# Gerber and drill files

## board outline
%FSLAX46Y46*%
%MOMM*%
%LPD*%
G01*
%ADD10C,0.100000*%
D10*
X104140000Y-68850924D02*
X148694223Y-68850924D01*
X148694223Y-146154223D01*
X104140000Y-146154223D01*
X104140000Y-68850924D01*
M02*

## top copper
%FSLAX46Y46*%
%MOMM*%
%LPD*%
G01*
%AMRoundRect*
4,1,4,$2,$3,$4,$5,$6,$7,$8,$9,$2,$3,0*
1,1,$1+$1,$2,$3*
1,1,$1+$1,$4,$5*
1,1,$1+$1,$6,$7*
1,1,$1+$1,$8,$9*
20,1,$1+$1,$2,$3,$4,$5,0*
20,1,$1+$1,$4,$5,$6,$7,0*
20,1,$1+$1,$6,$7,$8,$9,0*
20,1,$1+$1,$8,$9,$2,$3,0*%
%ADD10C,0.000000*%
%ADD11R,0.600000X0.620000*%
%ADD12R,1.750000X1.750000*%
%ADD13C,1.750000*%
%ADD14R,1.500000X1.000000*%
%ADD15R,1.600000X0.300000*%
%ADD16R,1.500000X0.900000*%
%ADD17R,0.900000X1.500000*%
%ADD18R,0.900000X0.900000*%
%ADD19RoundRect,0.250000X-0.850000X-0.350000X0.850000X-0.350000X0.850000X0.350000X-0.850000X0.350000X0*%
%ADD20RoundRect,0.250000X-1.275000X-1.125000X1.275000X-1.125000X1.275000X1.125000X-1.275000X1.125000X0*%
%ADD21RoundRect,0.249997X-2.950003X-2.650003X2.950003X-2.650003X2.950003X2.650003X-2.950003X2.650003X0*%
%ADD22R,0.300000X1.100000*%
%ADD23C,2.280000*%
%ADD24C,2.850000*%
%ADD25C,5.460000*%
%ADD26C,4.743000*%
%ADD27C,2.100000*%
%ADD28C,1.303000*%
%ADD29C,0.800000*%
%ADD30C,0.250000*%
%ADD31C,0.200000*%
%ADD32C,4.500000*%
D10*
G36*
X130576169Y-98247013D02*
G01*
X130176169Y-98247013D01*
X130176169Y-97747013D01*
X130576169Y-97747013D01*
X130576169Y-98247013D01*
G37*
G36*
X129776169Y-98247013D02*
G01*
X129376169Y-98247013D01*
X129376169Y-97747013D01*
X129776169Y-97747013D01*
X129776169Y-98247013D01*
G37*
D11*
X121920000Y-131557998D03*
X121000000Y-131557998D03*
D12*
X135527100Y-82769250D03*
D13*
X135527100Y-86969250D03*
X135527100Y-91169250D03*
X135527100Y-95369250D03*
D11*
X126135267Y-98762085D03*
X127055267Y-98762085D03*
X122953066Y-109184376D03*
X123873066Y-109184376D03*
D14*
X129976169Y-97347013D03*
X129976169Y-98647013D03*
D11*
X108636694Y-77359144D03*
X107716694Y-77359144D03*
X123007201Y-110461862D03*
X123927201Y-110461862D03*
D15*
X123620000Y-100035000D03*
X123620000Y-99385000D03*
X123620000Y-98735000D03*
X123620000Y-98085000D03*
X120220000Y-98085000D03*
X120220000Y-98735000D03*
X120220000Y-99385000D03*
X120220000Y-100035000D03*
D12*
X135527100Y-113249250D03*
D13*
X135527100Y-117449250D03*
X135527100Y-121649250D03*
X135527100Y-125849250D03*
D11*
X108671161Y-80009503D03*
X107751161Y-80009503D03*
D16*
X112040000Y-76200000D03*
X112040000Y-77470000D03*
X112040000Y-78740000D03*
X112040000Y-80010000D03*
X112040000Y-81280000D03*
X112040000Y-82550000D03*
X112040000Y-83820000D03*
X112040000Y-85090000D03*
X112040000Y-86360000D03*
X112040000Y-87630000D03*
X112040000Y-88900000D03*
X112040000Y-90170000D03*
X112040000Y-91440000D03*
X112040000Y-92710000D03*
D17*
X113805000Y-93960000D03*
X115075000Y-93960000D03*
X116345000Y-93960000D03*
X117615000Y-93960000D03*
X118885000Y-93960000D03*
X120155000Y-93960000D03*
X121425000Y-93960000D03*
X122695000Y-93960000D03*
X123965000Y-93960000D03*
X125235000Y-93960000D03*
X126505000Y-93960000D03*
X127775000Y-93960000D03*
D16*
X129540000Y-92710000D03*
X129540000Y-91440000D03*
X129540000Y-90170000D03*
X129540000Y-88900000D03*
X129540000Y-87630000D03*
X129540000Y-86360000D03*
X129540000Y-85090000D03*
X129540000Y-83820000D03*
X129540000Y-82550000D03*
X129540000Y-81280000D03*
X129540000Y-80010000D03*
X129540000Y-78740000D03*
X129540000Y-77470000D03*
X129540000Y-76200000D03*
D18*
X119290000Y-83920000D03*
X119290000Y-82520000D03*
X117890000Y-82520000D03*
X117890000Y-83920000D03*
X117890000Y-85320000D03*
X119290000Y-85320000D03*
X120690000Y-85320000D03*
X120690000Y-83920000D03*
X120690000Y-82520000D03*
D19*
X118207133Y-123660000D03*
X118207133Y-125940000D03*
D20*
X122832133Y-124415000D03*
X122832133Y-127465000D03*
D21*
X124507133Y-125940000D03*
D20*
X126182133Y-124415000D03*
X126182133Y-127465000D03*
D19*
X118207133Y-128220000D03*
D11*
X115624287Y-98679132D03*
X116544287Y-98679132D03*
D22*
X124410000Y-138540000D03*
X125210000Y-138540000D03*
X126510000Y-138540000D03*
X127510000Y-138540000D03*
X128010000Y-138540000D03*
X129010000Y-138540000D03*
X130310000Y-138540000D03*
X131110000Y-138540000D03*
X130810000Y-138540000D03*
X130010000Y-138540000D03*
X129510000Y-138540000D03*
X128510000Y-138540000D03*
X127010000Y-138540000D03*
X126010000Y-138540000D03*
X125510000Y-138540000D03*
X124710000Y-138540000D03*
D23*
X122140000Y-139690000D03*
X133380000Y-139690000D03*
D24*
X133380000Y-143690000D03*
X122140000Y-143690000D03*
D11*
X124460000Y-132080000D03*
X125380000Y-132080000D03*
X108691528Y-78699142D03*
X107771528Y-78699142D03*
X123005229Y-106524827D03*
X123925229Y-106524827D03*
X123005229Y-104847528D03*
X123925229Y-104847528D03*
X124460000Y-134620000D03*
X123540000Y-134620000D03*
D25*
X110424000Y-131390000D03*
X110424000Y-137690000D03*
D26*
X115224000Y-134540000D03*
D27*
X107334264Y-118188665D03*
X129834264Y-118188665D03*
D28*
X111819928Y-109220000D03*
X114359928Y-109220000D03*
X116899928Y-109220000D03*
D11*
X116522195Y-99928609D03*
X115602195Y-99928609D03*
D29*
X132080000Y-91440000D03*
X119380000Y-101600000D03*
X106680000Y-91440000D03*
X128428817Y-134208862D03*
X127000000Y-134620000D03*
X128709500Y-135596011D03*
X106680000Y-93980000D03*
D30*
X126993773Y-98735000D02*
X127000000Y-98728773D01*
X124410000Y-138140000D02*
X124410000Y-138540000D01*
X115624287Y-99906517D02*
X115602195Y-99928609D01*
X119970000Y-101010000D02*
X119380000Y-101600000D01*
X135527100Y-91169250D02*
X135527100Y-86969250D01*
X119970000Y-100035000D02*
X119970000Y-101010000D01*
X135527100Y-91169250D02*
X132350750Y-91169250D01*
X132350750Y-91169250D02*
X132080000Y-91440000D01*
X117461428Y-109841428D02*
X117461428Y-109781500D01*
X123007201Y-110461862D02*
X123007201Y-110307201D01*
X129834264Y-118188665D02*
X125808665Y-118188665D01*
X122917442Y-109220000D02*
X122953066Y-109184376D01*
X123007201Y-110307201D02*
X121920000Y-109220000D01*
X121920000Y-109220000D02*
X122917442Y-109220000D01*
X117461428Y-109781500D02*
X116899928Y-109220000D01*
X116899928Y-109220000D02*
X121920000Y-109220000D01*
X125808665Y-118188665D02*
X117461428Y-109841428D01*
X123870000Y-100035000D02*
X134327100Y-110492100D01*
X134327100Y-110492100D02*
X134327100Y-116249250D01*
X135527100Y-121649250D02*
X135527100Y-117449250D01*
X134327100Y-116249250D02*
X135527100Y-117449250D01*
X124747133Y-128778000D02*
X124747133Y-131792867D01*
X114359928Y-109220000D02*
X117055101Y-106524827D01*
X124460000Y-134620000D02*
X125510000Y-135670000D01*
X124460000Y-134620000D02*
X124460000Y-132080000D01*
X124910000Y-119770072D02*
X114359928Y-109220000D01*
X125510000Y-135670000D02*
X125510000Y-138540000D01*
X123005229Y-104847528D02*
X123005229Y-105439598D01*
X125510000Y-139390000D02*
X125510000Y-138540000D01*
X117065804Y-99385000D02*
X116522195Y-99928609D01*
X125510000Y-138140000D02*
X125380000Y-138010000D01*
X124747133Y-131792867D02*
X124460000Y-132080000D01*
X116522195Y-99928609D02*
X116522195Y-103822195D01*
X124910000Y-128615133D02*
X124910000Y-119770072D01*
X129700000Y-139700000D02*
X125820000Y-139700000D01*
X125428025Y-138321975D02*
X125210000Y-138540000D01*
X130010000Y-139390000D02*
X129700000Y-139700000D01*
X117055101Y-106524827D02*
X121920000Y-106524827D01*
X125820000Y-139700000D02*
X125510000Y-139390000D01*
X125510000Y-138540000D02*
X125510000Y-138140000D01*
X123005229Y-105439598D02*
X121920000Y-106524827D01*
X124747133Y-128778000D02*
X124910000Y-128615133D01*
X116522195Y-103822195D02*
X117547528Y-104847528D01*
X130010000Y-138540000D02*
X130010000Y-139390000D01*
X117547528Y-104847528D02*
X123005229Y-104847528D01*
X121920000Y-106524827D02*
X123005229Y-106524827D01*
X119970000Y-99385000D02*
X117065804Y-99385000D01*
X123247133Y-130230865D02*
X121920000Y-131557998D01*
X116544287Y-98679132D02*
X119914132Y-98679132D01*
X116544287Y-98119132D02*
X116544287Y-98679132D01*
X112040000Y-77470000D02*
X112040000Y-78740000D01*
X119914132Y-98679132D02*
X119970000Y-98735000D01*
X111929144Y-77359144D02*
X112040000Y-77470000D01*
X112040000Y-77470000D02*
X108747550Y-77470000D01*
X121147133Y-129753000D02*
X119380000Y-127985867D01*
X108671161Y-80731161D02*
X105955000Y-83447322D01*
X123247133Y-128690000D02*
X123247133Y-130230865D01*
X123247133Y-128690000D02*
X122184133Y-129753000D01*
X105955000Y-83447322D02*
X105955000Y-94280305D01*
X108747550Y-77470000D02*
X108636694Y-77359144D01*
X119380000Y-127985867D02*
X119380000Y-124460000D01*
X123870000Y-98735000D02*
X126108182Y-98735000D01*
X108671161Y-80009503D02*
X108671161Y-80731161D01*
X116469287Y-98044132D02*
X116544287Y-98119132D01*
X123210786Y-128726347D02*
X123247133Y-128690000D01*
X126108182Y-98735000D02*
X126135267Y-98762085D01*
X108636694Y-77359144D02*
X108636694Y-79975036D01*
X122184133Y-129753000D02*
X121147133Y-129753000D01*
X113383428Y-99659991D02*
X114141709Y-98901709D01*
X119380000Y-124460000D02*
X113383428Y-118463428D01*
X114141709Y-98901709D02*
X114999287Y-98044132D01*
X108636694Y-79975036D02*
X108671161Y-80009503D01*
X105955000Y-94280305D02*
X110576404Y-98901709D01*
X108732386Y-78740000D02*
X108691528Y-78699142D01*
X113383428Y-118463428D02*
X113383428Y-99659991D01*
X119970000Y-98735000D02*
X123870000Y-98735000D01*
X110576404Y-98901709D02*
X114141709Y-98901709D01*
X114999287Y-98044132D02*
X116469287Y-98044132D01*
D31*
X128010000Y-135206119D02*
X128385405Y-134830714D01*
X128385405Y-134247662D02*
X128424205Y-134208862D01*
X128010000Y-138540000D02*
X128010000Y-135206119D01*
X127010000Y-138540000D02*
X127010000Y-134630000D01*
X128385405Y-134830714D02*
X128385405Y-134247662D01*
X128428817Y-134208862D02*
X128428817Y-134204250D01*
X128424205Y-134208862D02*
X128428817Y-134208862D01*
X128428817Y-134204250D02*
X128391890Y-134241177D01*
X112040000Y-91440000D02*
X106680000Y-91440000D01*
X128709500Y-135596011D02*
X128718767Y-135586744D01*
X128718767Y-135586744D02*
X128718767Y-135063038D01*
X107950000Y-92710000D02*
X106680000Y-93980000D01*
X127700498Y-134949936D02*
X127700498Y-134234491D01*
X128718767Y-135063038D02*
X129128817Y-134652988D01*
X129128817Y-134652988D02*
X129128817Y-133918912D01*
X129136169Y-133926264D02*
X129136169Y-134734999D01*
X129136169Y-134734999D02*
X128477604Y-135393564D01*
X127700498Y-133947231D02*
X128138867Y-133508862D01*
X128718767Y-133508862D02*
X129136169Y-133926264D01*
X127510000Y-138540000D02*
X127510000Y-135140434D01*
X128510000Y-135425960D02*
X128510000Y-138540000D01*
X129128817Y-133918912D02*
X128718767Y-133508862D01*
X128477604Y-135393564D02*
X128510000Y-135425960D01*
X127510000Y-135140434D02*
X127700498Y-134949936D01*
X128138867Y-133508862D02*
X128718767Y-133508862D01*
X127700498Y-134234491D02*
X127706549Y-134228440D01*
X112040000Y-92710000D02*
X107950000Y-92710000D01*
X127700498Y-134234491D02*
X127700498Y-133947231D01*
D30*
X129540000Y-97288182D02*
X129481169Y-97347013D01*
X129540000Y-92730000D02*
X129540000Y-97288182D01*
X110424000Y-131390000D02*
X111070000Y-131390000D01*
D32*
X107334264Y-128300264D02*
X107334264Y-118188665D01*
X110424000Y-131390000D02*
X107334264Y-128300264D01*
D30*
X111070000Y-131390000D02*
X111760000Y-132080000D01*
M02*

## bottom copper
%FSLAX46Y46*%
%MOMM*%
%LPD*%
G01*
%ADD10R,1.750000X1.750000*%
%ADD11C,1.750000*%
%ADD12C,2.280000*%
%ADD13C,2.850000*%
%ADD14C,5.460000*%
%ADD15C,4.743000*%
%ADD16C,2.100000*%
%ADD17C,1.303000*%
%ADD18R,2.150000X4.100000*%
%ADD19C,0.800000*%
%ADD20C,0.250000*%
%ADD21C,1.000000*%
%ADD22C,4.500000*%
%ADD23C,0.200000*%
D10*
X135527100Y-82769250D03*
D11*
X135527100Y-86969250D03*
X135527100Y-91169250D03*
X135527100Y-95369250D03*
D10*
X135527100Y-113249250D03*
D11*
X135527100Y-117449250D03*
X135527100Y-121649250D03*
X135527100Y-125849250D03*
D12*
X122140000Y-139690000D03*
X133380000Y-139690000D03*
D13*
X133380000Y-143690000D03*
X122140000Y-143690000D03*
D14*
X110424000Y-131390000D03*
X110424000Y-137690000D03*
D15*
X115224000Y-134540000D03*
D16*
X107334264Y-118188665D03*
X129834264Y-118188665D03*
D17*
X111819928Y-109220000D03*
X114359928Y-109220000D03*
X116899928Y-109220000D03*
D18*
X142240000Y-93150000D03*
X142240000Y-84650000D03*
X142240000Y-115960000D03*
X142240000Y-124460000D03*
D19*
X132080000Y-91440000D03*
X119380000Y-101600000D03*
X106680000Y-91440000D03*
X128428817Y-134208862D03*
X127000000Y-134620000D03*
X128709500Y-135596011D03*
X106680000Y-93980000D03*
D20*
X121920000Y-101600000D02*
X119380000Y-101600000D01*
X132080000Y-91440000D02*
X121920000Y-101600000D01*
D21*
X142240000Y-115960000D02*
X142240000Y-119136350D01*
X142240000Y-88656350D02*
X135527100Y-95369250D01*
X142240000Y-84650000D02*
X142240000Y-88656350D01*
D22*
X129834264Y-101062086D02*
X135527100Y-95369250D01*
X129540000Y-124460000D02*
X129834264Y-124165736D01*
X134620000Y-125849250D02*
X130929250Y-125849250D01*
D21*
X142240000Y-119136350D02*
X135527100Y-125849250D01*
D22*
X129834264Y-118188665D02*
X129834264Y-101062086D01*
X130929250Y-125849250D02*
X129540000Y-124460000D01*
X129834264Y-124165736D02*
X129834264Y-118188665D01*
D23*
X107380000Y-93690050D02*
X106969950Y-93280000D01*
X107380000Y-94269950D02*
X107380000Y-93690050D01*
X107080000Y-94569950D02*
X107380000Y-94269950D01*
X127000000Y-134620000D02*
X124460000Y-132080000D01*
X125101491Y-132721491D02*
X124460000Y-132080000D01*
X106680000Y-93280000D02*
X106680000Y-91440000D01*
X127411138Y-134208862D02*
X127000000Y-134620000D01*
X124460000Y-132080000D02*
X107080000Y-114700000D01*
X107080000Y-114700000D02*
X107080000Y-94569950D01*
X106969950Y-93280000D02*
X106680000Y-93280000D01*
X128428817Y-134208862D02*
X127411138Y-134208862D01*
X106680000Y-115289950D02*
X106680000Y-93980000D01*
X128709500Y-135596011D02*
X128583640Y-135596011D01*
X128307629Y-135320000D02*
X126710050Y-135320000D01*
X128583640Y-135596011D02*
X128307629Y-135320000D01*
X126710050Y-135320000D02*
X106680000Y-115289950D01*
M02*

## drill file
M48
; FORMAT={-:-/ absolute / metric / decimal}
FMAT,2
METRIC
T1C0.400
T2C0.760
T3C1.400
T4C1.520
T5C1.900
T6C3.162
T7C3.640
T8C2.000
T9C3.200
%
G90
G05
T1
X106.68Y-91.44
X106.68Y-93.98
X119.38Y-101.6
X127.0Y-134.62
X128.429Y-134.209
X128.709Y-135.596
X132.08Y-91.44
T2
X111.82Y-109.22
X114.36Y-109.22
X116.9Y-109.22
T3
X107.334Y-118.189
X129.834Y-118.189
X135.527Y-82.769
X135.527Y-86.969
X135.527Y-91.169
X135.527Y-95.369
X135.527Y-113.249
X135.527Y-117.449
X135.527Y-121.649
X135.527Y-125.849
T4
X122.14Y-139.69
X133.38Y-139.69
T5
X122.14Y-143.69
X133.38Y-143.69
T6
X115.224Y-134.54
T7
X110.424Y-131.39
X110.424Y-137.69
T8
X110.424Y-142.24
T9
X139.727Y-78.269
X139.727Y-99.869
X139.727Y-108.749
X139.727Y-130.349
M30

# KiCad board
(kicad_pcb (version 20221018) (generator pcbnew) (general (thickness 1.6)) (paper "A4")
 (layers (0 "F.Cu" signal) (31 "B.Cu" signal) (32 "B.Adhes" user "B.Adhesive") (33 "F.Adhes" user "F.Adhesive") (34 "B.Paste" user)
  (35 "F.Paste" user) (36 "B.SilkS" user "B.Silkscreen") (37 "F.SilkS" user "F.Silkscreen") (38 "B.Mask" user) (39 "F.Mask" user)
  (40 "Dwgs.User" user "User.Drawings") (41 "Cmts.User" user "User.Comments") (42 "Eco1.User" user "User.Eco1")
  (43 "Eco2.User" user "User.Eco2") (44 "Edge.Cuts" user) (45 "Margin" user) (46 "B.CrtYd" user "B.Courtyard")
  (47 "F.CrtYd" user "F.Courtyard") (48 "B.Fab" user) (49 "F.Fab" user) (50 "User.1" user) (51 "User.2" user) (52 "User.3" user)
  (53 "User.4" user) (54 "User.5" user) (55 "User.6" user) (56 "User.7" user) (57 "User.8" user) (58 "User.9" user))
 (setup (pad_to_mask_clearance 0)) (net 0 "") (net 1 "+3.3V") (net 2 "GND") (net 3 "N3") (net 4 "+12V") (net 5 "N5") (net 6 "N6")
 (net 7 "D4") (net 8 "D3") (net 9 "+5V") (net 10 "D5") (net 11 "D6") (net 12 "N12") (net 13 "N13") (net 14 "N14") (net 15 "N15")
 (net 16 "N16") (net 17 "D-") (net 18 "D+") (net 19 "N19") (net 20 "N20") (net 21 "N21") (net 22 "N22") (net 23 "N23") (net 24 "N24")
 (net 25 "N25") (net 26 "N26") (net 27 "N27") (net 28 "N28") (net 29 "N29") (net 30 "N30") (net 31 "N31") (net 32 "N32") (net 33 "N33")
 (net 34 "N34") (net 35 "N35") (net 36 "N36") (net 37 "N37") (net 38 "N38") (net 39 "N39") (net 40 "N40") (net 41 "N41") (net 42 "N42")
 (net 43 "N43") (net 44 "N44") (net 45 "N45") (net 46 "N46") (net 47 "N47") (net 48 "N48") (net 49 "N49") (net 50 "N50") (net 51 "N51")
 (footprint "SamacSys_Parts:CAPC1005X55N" (layer "F.Cu") (at 121.46 131.557998 180)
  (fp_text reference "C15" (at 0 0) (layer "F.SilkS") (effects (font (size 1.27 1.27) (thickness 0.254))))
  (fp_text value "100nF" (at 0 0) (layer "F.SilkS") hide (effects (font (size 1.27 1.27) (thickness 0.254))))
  (pad "1" smd rect (at -0.46 0 180) (size 0.6 0.62) (layers "F.Cu" "F.Paste" "F.Mask") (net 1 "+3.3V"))
  (pad "2" smd rect (at 0.46 0 180) (size 0.6 0.62) (layers "F.Cu" "F.Paste" "F.Mask") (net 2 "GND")))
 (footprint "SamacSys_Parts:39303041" (layer "F.Cu") (at 135.5271 82.76925 90)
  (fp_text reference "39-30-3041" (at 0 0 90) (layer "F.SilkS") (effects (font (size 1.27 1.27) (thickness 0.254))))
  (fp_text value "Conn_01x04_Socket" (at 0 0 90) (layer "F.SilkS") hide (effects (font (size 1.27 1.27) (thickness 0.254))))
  (pad "" np_thru_hole circle (at -17.1 4.2 90) (size 3.2 3.2) (drill 3.2) (layers "*.Cu" "*.Mask"))
  (pad "" np_thru_hole circle (at 4.5 4.2 90) (size 3.2 3.2) (drill 3.2) (layers "*.Cu" "*.Mask"))
  (pad "1" thru_hole rect (at 0 0 90) (size 1.75 1.75) (drill 1.4) (layers "*.Cu" "*.Mask") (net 2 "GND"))
  (pad "2" thru_hole circle (at -4.2 0 90) (size 1.75 1.75) (drill 1.4) (layers "*.Cu" "*.Mask") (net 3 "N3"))
  (pad "3" thru_hole circle (at -8.4 0 90) (size 1.75 1.75) (drill 1.4) (layers "*.Cu" "*.Mask") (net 3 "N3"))
  (pad "4" thru_hole circle (at -12.6 0 90) (size 1.75 1.75) (drill 1.4) (layers "*.Cu" "*.Mask") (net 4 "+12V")))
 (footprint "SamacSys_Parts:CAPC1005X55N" (layer "F.Cu") (at 126.595267 98.762085)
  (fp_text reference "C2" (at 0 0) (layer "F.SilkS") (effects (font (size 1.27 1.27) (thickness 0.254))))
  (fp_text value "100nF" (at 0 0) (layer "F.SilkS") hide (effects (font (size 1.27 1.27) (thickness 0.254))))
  (pad "1" smd rect (at -0.46 0) (size 0.6 0.62) (layers "F.Cu" "F.Paste" "F.Mask") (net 1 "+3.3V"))
  (pad "2" smd rect (at 0.46 0) (size 0.6 0.62) (layers "F.Cu" "F.Paste" "F.Mask") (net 2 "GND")))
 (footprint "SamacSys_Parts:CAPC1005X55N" (layer "F.Cu") (at 123.413066 109.184376)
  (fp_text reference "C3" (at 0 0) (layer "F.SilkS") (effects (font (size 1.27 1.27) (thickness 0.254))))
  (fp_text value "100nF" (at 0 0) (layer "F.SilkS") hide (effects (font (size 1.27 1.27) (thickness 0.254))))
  (pad "1" smd rect (at -0.46 0) (size 0.6 0.62) (layers "F.Cu" "F.Paste" "F.Mask") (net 4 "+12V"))
  (pad "2" smd rect (at 0.46 0) (size 0.6 0.62) (layers "F.Cu" "F.Paste" "F.Mask") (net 2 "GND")))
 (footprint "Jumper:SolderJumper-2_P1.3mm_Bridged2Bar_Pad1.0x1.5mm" (layer "F.Cu") (at 129.976169 97.997013 -90) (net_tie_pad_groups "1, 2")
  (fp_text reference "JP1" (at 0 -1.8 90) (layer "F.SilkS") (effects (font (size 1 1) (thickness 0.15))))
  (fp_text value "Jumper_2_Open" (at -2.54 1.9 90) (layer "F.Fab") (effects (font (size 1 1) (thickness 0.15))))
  (fp_poly (pts (xy -0.25 -0.6) (xy 0.25 -0.6) (xy 0.25 -0.2) (xy -0.25 -0.2)) (stroke (width 0) (type solid)) (fill solid) (layer "F.Cu"))
  (fp_poly (pts (xy -0.25 0.2) (xy 0.25 0.2) (xy 0.25 0.6) (xy -0.25 0.6)) (stroke (width 0) (type solid)) (fill solid) (layer "F.Cu"))
  (pad "1" smd rect (at -0.65 0 270) (size 1 1.5) (layers "F.Cu" "F.Mask") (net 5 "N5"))
  (pad "2" smd rect (at 0.65 0 270) (size 1 1.5) (layers "F.Cu" "F.Mask") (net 2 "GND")))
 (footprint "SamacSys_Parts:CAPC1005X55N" (layer "F.Cu") (at 108.176694 77.359144 180)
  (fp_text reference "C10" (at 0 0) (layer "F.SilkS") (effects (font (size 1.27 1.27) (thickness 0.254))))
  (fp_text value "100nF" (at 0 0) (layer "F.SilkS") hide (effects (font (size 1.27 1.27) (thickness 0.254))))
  (pad "1" smd rect (at -0.46 0 180) (size 0.6 0.62) (layers "F.Cu" "F.Paste" "F.Mask") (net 1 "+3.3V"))
  (pad "2" smd rect (at 0.46 0 180) (size 0.6 0.62) (layers "F.Cu" "F.Paste" "F.Mask") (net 2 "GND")))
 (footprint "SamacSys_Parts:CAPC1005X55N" (layer "F.Cu") (at 123.467201 110.461862)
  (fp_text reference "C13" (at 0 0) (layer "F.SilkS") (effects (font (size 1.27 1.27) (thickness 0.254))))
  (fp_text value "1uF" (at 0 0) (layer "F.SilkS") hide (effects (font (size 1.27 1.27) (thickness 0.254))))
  (pad "1" smd rect (at -0.46 0) (size 0.6 0.62) (layers "F.Cu" "F.Paste" "F.Mask") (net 4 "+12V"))
  (pad "2" smd rect (at 0.46 0) (size 0.6 0.62) (layers "F.Cu" "F.Paste" "F.Mask") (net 2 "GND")))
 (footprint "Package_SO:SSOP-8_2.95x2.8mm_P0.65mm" (layer "F.Cu") (at 121.92 99.06 180)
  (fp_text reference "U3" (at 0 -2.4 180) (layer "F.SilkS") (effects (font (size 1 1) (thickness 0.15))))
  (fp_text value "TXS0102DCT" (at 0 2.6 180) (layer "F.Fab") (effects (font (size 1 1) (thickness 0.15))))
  (pad "1" smd rect (at -1.7 -0.975 90) (size 0.3 1.6) (layers "F.Cu" "F.Paste" "F.Mask") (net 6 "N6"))
  (pad "2" smd rect (at -1.7 -0.325 90) (size 0.3 1.6) (layers "F.Cu" "F.Paste" "F.Mask") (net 2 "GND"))
  (pad "3" smd rect (at -1.7 0.325 90) (size 0.3 1.6) (layers "F.Cu" "F.Paste" "F.Mask") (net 1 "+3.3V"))
  (pad "4" smd rect (at -1.7 0.975 90) (size 0.3 1.6) (layers "F.Cu" "F.Paste" "F.Mask") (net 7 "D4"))
  (pad "5" smd rect (at 1.7 0.975 90) (size 0.3 1.6) (layers "F.Cu" "F.Paste" "F.Mask") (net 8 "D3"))
  (pad "6" smd rect (at 1.7 0.325 90) (size 0.3 1.6) (layers "F.Cu" "F.Paste" "F.Mask") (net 1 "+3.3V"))
  (pad "7" smd rect (at 1.7 -0.325 90) (size 0.3 1.6) (layers "F.Cu" "F.Paste" "F.Mask") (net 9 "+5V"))
  (pad "8" smd rect (at 1.7 -0.975 90) (size 0.3 1.6) (layers "F.Cu" "F.Paste" "F.Mask") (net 3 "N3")))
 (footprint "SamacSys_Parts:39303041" (layer "F.Cu") (at 135.5271 113.24925 90)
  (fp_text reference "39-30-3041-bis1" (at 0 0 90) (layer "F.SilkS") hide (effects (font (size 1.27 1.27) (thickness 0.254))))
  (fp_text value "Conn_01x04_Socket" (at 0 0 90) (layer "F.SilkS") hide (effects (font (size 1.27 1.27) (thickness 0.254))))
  (pad "" np_thru_hole circle (at -17.1 4.2 90) (size 3.2 3.2) (drill 3.2) (layers "*.Cu" "*.Mask"))
  (pad "" np_thru_hole circle (at 4.5 4.2 90) (size 3.2 3.2) (drill 3.2) (layers "*.Cu" "*.Mask"))
  (pad "1" thru_hole rect (at 0 0 90) (size 1.75 1.75) (drill 1.4) (layers "*.Cu" "*.Mask") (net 2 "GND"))
  (pad "2" thru_hole circle (at -4.2 0 90) (size 1.75 1.75) (drill 1.4) (layers "*.Cu" "*.Mask") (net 6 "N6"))
  (pad "3" thru_hole circle (at -8.4 0 90) (size 1.75 1.75) (drill 1.4) (layers "*.Cu" "*.Mask") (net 6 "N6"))
  (pad "4" thru_hole circle (at -12.6 0 90) (size 1.75 1.75) (drill 1.4) (layers "*.Cu" "*.Mask") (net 4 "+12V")))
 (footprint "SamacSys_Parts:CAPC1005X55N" (layer "F.Cu") (at 108.211161 80.009503 180)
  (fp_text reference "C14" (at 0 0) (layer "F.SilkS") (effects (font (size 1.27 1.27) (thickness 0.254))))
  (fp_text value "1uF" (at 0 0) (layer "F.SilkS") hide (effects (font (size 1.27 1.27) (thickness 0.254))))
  (pad "1" smd rect (at -0.46 0 180) (size 0.6 0.62) (layers "F.Cu" "F.Paste" "F.Mask") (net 1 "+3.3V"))
  (pad "2" smd rect (at 0.46 0 180) (size 0.6 0.62) (layers "F.Cu" "F.Paste" "F.Mask") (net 2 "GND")))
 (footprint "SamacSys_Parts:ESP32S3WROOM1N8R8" (layer "F.Cu") (at 120.79 81.46)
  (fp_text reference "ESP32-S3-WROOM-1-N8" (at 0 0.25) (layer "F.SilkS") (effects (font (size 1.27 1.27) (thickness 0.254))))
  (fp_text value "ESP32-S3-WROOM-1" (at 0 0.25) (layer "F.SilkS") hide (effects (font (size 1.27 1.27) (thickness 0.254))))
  (pad "1" smd rect (at -8.75 -5.26 90) (size 0.9 1.5) (layers "F.Cu" "F.Paste" "F.Mask") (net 2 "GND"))
  (pad "2" smd rect (at -8.75 -3.99 90) (size 0.9 1.5) (layers "F.Cu" "F.Paste" "F.Mask") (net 1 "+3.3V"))
  (pad "3" smd rect (at -8.75 -2.72 90) (size 0.9 1.5) (layers "F.Cu" "F.Paste" "F.Mask") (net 1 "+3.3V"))
  (pad "4" smd rect (at -8.75 -1.45 90) (size 0.9 1.5) (layers "F.Cu" "F.Paste" "F.Mask") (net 8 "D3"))
  (pad "5" smd rect (at -8.75 -0.18 90) (size 0.9 1.5) (layers "F.Cu" "F.Paste" "F.Mask") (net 7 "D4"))
  (pad "6" smd rect (at -8.75 1.09 90) (size 0.9 1.5) (layers "F.Cu" "F.Paste" "F.Mask") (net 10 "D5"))
  (pad "7" smd rect (at -8.75 2.36 90) (size 0.9 1.5) (layers "F.Cu" "F.Paste" "F.Mask") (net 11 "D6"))
  (pad "8" smd rect (at -8.75 3.63 90) (size 0.9 1.5) (layers "F.Cu" "F.Paste" "F.Mask") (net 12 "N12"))
  (pad "9" smd rect (at -8.75 4.9 90) (size 0.9 1.5) (layers "F.Cu" "F.Paste" "F.Mask") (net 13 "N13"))
  (pad "10" smd rect (at -8.75 6.17 90) (size 0.9 1.5) (layers "F.Cu" "F.Paste" "F.Mask") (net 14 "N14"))
  (pad "11" smd rect (at -8.75 7.44 90) (size 0.9 1.5) (layers "F.Cu" "F.Paste" "F.Mask") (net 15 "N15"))
  (pad "12" smd rect (at -8.75 8.71 90) (size 0.9 1.5) (layers "F.Cu" "F.Paste" "F.Mask") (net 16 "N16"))
  (pad "13" smd rect (at -8.75 9.98 90) (size 0.9 1.5) (layers "F.Cu" "F.Paste" "F.Mask") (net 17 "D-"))
  (pad "14" smd rect (at -8.75 11.25 90) (size 0.9 1.5) (layers "F.Cu" "F.Paste" "F.Mask") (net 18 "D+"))
  (pad "15" smd rect (at -6.985 12.5) (size 0.9 1.5) (layers "F.Cu" "F.Paste" "F.Mask") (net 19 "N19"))
  (pad "16" smd rect (at -5.715 12.5) (size 0.9 1.5) (layers "F.Cu" "F.Paste" "F.Mask") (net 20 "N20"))
  (pad "17" smd rect (at -4.445 12.5) (size 0.9 1.5) (layers "F.Cu" "F.Paste" "F.Mask") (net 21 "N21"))
  (pad "18" smd rect (at -3.175 12.5) (size 0.9 1.5) (layers "F.Cu" "F.Paste" "F.Mask") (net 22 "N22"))
  (pad "19" smd rect (at -1.905 12.5) (size 0.9 1.5) (layers "F.Cu" "F.Paste" "F.Mask") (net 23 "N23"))
  (pad "20" smd rect (at -0.635 12.5) (size 0.9 1.5) (layers "F.Cu" "F.Paste" "F.Mask") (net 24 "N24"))
  (pad "21" smd rect (at 0.635 12.5) (size 0.9 1.5) (layers "F.Cu" "F.Paste" "F.Mask") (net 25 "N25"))
  (pad "22" smd rect (at 1.905 12.5) (size 0.9 1.5) (layers "F.Cu" "F.Paste" "F.Mask") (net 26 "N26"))
  (pad "23" smd rect (at 3.175 12.5) (size 0.9 1.5) (layers "F.Cu" "F.Paste" "F.Mask") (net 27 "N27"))
  (pad "24" smd rect (at 4.445 12.5) (size 0.9 1.5) (layers "F.Cu" "F.Paste" "F.Mask") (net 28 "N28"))
  (pad "25" smd rect (at 5.715 12.5) (size 0.9 1.5) (layers "F.Cu" "F.Paste" "F.Mask") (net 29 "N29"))
  (pad "26" smd rect (at 6.985 12.5) (size 0.9 1.5) (layers "F.Cu" "F.Paste" "F.Mask") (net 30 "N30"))
  (pad "27" smd rect (at 8.75 11.25 90) (size 0.9 1.5) (layers "F.Cu" "F.Paste" "F.Mask") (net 5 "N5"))
  (pad "28" smd rect (at 8.75 9.98 90) (size 0.9 1.5) (layers "F.Cu" "F.Paste" "F.Mask") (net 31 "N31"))
  (pad "29" smd rect (at 8.75 8.71 90) (size 0.9 1.5) (layers "F.Cu" "F.Paste" "F.Mask") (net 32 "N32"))
  (pad "30" smd rect (at 8.75 7.44 90) (size 0.9 1.5) (layers "F.Cu" "F.Paste" "F.Mask") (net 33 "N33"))
  (pad "31" smd rect (at 8.75 6.17 90) (size 0.9 1.5) (layers "F.Cu" "F.Paste" "F.Mask") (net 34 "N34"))
  (pad "32" smd rect (at 8.75 4.9 90) (size 0.9 1.5) (layers "F.Cu" "F.Paste" "F.Mask") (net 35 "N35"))
  (pad "33" smd rect (at 8.75 3.63 90) (size 0.9 1.5) (layers "F.Cu" "F.Paste" "F.Mask") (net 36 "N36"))
  (pad "34" smd rect (at 8.75 2.36 90) (size 0.9 1.5) (layers "F.Cu" "F.Paste" "F.Mask") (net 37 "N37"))
  (pad "35" smd rect (at 8.75 1.09 90) (size 0.9 1.5) (layers "F.Cu" "F.Paste" "F.Mask") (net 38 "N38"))
  (pad "36" smd rect (at 8.75 -0.18 90) (size 0.9 1.5) (layers "F.Cu" "F.Paste" "F.Mask") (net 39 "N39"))
  (pad "37" smd rect (at 8.75 -1.45 90) (size 0.9 1.5) (layers "F.Cu" "F.Paste" "F.Mask") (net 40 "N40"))
  (pad "38" smd rect (at 8.75 -2.72 90) (size 0.9 1.5) (layers "F.Cu" "F.Paste" "F.Mask") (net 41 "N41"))
  (pad "39" smd rect (at 8.75 -3.99 90) (size 0.9 1.5) (layers "F.Cu" "F.Paste" "F.Mask") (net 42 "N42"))
  (pad "40" smd rect (at 8.75 -5.26 90) (size 0.9 1.5) (layers "F.Cu" "F.Paste" "F.Mask") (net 2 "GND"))
  (pad "41" smd rect (at -1.5 2.46) (size 0.9 0.9) (layers "F.Cu" "F.Paste" "F.Mask") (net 2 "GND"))
  (pad "42" smd rect (at -1.5 1.06) (size 0.9 0.9) (layers "F.Cu" "F.Paste" "F.Mask"))
  (pad "43" smd rect (at -2.9 1.06) (size 0.9 0.9) (layers "F.Cu" "F.Paste" "F.Mask"))
  (pad "44" smd rect (at -2.9 2.46) (size 0.9 0.9) (layers "F.Cu" "F.Paste" "F.Mask"))
  (pad "45" smd rect (at -2.9 3.86) (size 0.9 0.9) (layers "F.Cu" "F.Paste" "F.Mask"))
  (pad "46" smd rect (at -1.5 3.86) (size 0.9 0.9) (layers "F.Cu" "F.Paste" "F.Mask"))
  (pad "47" smd rect (at -0.1 3.86) (size 0.9 0.9) (layers "F.Cu" "F.Paste" "F.Mask"))
  (pad "48" smd rect (at -0.1 2.46) (size 0.9 0.9) (layers "F.Cu" "F.Paste" "F.Mask"))
  (pad "49" smd rect (at -0.1 1.06) (size 0.9 0.9) (layers "F.Cu" "F.Paste" "F.Mask")))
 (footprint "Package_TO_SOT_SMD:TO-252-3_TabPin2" (layer "F.Cu") (at 123.247133 125.94)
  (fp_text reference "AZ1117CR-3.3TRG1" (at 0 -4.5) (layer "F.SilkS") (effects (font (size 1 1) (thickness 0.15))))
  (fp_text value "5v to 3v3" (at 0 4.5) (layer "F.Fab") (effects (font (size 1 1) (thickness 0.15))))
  (pad "1" smd roundrect (at -5.04 -2.28) (size 2.2 1.2) (layers "F.Cu" "F.Paste" "F.Mask") (roundrect_rratio 0.208333) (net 2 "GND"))
  (pad "2" smd roundrect (at -5.04 0) (size 2.2 1.2) (layers "F.Cu" "F.Paste" "F.Mask") (roundrect_rratio 0.208333) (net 1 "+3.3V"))
  (pad "2" smd roundrect (at -0.415 -1.525) (size 3.05 2.75) (layers "F.Cu" "F.Paste") (roundrect_rratio 0.090909) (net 1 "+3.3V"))
  (pad "2" smd roundrect (at -0.415 1.525) (size 3.05 2.75) (layers "F.Cu" "F.Paste") (roundrect_rratio 0.090909) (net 1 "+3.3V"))
  (pad "2" smd roundrect (at 1.26 0) (size 6.4 5.8) (layers "F.Cu" "F.Mask") (roundrect_rratio 0.043103) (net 1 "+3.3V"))
  (pad "2" smd roundrect (at 2.935 -1.525) (size 3.05 2.75) (layers "F.Cu" "F.Paste") (roundrect_rratio 0.090909) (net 1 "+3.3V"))
  (pad "2" smd roundrect (at 2.935 1.525) (size 3.05 2.75) (layers "F.Cu" "F.Paste") (roundrect_rratio 0.090909) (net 1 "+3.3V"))
  (pad "3" smd roundrect (at -5.04 2.28) (size 2.2 1.2) (layers "F.Cu" "F.Paste" "F.Mask") (roundrect_rratio 0.208333) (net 9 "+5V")))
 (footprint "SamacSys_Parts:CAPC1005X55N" (layer "F.Cu") (at 116.084287 98.679132)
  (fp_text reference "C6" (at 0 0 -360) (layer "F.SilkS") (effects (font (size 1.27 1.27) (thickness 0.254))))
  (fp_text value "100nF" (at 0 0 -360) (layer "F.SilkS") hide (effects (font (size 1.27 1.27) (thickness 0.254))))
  (pad "1" smd rect (at -0.46 0) (size 0.6 0.62) (layers "F.Cu" "F.Paste" "F.Mask") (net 2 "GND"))
  (pad "2" smd rect (at 0.46 0) (size 0.6 0.62) (layers "F.Cu" "F.Paste" "F.Mask") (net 1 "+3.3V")))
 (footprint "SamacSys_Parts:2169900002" (layer "F.Cu") (at 127.76 141.39)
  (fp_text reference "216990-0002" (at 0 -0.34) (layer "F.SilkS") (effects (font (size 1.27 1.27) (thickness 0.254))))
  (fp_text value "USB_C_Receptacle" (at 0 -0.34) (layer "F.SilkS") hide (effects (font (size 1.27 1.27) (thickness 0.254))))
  (pad "A1" smd rect (at -3.35 -2.85) (size 0.3 1.1) (layers "F.Cu" "F.Paste" "F.Mask") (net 2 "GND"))
  (pad "A4" smd rect (at -2.55 -2.85) (size 0.3 1.1) (layers "F.Cu" "F.Paste" "F.Mask") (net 9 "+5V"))
  (pad "A5" smd rect (at -1.25 -2.85) (size 0.3 1.1) (layers "F.Cu" "F.Paste" "F.Mask") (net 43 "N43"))
  (pad "A6" smd rect (at -0.25 -2.85) (size 0.3 1.1) (layers "F.Cu" "F.Paste" "F.Mask") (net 18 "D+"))
  (pad "A7" smd rect (at 0.25 -2.85) (size 0.3 1.1) (layers "F.Cu" "F.Paste" "F.Mask") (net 17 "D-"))
  (pad "A8" smd rect (at 1.25 -2.85) (size 0.3 1.1) (layers "F.Cu" "F.Paste" "F.Mask") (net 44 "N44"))
  (pad "A9" smd rect (at 2.55 -2.85) (size 0.3 1.1) (layers "F.Cu" "F.Paste" "F.Mask") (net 9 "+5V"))
  (pad "A12" smd rect (at 3.35 -2.85) (size 0.3 1.1) (layers "F.Cu" "F.Paste" "F.Mask") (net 2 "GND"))
  (pad "B1" smd rect (at 3.05 -2.85) (size 0.3 1.1) (layers "F.Cu" "F.Paste" "F.Mask") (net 2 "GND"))
  (pad "B4" smd rect (at 2.25 -2.85) (size 0.3 1.1) (layers "F.Cu" "F.Paste" "F.Mask") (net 9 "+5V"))
  (pad "B5" smd rect (at 1.75 -2.85) (size 0.3 1.1) (layers "F.Cu" "F.Paste" "F.Mask") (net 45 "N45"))
  (pad "B6" smd rect (at 0.75 -2.85) (size 0.3 1.1) (layers "F.Cu" "F.Paste" "F.Mask") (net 18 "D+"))
  (pad "B7" smd rect (at -0.75 -2.85) (size 0.3 1.1) (layers "F.Cu" "F.Paste" "F.Mask") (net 17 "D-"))
  (pad "B8" smd rect (at -1.75 -2.85) (size 0.3 1.1) (layers "F.Cu" "F.Paste" "F.Mask") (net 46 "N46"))
  (pad "B9" smd rect (at -2.25 -2.85) (size 0.3 1.1) (layers "F.Cu" "F.Paste" "F.Mask") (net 9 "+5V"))
  (pad "B12" smd rect (at -3.05 -2.85) (size 0.3 1.1) (layers "F.Cu" "F.Paste" "F.Mask") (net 2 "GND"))
  (pad "MH1" thru_hole circle (at -5.62 -1.7) (size 2.28 2.28) (drill 1.52) (layers "*.Cu" "*.Mask") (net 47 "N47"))
  (pad "MH2" thru_hole circle (at 5.62 -1.7) (size 2.28 2.28) (drill 1.52) (layers "*.Cu" "*.Mask") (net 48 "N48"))
  (pad "MH3" thru_hole circle (at 5.62 2.3) (size 2.85 2.85) (drill 1.9) (layers "*.Cu" "*.Mask") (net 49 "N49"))
  (pad "MH4" thru_hole circle (at -5.62 2.3) (size 2.85 2.85) (drill 1.9) (layers "*.Cu" "*.Mask") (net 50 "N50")))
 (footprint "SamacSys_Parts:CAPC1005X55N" (layer "F.Cu") (at 124.92 132.08)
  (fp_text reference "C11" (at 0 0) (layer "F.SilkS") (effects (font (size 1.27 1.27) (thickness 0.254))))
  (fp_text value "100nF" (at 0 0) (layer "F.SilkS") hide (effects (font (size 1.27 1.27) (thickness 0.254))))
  (pad "1" smd rect (at -0.46 0) (size 0.6 0.62) (layers "F.Cu" "F.Paste" "F.Mask") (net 9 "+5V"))
  (pad "2" smd rect (at 0.46 0) (size 0.6 0.62) (layers "F.Cu" "F.Paste" "F.Mask") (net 2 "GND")))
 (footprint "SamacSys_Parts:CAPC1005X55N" (layer "F.Cu") (at 108.231528 78.699142 180)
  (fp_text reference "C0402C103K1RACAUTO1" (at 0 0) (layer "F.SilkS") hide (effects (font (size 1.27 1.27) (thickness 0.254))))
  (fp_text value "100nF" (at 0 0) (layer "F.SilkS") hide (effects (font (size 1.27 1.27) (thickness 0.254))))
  (pad "1" smd rect (at -0.46 0 180) (size 0.6 0.62) (layers "F.Cu" "F.Paste" "F.Mask") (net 1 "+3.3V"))
  (pad "2" smd rect (at 0.46 0 180) (size 0.6 0.62) (layers "F.Cu" "F.Paste" "F.Mask") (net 2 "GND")))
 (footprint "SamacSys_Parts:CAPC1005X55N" (layer "F.Cu") (at 123.465229 106.524827)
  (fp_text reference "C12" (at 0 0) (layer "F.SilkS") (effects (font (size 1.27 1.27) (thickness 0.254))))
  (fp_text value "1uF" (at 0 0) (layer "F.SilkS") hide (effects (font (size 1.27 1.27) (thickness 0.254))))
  (pad "1" smd rect (at -0.46 0) (size 0.6 0.62) (layers "F.Cu" "F.Paste" "F.Mask") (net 9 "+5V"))
  (pad "2" smd rect (at 0.46 0) (size 0.6 0.62) (layers "F.Cu" "F.Paste" "F.Mask") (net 2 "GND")))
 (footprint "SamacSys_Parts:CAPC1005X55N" (layer "F.Cu") (at 123.465229 104.847528)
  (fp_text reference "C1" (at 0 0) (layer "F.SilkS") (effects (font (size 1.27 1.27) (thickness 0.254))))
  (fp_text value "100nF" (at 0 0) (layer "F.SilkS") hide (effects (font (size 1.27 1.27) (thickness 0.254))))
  (pad "1" smd rect (at -0.46 0) (size 0.6 0.62) (layers "F.Cu" "F.Paste" "F.Mask") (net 9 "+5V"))
  (pad "2" smd rect (at 0.46 0) (size 0.6 0.62) (layers "F.Cu" "F.Paste" "F.Mask") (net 2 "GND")))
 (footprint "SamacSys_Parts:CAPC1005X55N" (layer "F.Cu") (at 124 134.62 180)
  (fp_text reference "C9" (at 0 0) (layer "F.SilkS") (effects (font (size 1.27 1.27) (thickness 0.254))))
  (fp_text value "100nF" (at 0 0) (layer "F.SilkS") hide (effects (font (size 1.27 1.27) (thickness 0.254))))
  (pad "1" smd rect (at -0.46 0 180) (size 0.6 0.62) (layers "F.Cu" "F.Paste" "F.Mask") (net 9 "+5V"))
  (pad "2" smd rect (at 0.46 0 180) (size 0.6 0.62) (layers "F.Cu" "F.Paste" "F.Mask") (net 2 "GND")))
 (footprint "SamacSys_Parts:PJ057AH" (layer "F.Cu") (at 110.424 131.39 90)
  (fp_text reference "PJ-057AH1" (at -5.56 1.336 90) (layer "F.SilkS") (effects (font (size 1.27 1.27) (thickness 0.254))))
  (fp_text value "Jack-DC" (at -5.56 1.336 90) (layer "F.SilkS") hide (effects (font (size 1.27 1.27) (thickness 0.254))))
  (pad "" np_thru_hole circle (at -10.85 0 90) (size 2 2) (drill 2) (layers "*.Cu" "*.Mask"))
  (pad "1" thru_hole circle (at 0 0 90) (size 5.46 5.46) (drill 3.6401) (layers "*.Cu" "*.Mask") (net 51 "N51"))
  (pad "2" thru_hole circle (at -6.3 0 90) (size 5.46 5.46) (drill 3.6401) (layers "*.Cu" "*.Mask") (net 2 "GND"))
  (pad "3" thru_hole circle (at -3.15 4.8 90) (size 4.743 4.743) (drill 3.1623) (layers "*.Cu" "*.Mask")))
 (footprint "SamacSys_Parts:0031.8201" (layer "F.Cu") (at 118.584264 118.188665)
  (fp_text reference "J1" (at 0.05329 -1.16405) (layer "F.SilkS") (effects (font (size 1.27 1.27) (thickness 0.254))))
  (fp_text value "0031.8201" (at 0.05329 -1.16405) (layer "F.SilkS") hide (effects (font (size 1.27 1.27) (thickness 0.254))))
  (pad "1" thru_hole circle (at -11.25 0) (size 2.1 2.1) (drill 1.4) (layers "*.Cu" "*.Mask") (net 51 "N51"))
  (pad "2" thru_hole circle (at 11.25 0) (size 2.1 2.1) (drill 1.4) (layers "*.Cu" "*.Mask") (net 4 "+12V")))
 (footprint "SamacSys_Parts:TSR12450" (layer "F.Cu") (at 111.819928 109.22)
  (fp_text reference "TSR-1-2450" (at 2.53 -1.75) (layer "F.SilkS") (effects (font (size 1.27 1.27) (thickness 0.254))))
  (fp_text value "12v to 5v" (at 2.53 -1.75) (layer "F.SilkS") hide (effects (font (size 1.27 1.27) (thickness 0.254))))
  (pad "1" thru_hole circle (at 0 0) (size 1.303 1.303) (drill 0.76) (layers "*.Cu" "*.Mask") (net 2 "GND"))
  (pad "2" thru_hole circle (at 2.54 0) (size 1.303 1.303) (drill 0.76) (layers "*.Cu" "*.Mask") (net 9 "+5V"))
  (pad "3" thru_hole circle (at 5.08 0) (size 1.303 1.303) (drill 0.76) (layers "*.Cu" "*.Mask") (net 4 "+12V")))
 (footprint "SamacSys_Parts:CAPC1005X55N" (layer "F.Cu") (at 116.062195 99.928609 180)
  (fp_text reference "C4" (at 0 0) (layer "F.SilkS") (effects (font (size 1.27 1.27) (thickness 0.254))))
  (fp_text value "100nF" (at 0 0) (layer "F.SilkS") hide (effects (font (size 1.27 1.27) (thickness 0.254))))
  (pad "1" smd rect (at -0.46 0 180) (size 0.6 0.62) (layers "F.Cu" "F.Paste" "F.Mask") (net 9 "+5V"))
  (pad "2" smd rect (at 0.46 0 180) (size 0.6 0.62) (layers "F.Cu" "F.Paste" "F.Mask") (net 2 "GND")))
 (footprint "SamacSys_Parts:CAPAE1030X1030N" (layer "B.Cu") (at 142.24 88.9 90)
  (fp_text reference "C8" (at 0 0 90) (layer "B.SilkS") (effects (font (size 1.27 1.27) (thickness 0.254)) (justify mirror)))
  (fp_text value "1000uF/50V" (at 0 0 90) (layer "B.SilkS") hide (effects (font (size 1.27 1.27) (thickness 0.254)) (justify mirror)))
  (pad "1" smd rect (at -4.25 0) (size 2.15 4.1) (layers "B.Cu" "B.Paste" "B.Mask") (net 2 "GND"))
  (pad "2" smd rect (at 4.25 0) (size 2.15 4.1) (layers "B.Cu" "B.Paste" "B.Mask") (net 4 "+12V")))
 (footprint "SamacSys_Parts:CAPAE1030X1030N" (layer "B.Cu") (at 142.24 120.21 -90)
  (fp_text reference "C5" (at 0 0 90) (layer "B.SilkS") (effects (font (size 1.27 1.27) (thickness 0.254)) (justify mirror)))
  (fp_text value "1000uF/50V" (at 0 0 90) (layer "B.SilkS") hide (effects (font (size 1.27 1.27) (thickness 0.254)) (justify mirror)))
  (pad "1" smd rect (at -4.25 0 180) (size 2.15 4.1) (layers "B.Cu" "B.Paste" "B.Mask") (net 4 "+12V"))
  (pad "2" smd rect (at 4.25 0 180) (size 2.15 4.1) (layers "B.Cu" "B.Paste" "B.Mask") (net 2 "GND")))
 (gr_rect (start 104.14 68.850924) (end 148.694223 146.154223) (stroke (width 0.1) (type default)) (fill none) (layer "Edge.Cuts"))
 (segment (start 126.993773 98.735) (end 127 98.728773) (width 0.25) (layer "F.Cu") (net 2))
 (segment (start 124.41 138.14) (end 124.41 138.54) (width 0.25) (layer "F.Cu") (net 2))
 (segment (start 115.624287 99.906517) (end 115.602195 99.928609) (width 0.25) (layer "F.Cu") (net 2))
 (segment (start 119.97 101.01) (end 119.38 101.6) (width 0.25) (layer "F.Cu") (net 3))
 (segment (start 135.5271 91.16925) (end 135.5271 86.96925) (width 0.25) (layer "F.Cu") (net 3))
 (segment (start 119.97 100.035) (end 119.97 101.01) (width 0.25) (layer "F.Cu") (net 3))
 (segment (start 135.5271 91.16925) (end 132.35075 91.16925) (width 0.25) (layer "F.Cu") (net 3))
 (segment (start 132.35075 91.16925) (end 132.08 91.44) (width 0.25) (layer "F.Cu") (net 3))
 (via (at 132.08 91.44) (size 0.8) (drill 0.4) (layers "F.Cu" "B.Cu") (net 3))
 (via (at 119.38 101.6) (size 0.8) (drill 0.4) (layers "F.Cu" "B.Cu") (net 3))
 (segment (start 121.92 101.6) (end 119.38 101.6) (width 0.25) (layer "B.Cu") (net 3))
 (segment (start 132.08 91.44) (end 121.92 101.6) (width 0.25) (layer "B.Cu") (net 3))
 (segment (start 117.461428 109.841428) (end 117.461428 109.7815) (width 0.25) (layer "F.Cu") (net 4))
 (segment (start 123.007201 110.461862) (end 123.007201 110.307201) (width 0.25) (layer "F.Cu") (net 4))
 (segment (start 129.834264 118.188665) (end 125.808665 118.188665) (width 0.25) (layer "F.Cu") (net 4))
 (segment (start 122.917442 109.22) (end 122.953066 109.184376) (width 0.25) (layer "F.Cu") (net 4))
 (segment (start 123.007201 110.307201) (end 121.92 109.22) (width 0.25) (layer "F.Cu") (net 4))
 (segment (start 121.92 109.22) (end 122.917442 109.22) (width 0.25) (layer "F.Cu") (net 4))
 (segment (start 117.461428 109.7815) (end 116.899928 109.22) (width 0.25) (layer "F.Cu") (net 4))
 (segment (start 116.899928 109.22) (end 121.92 109.22) (width 0.25) (layer "F.Cu") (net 4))
 (segment (start 125.808665 118.188665) (end 117.461428 109.841428) (width 0.25) (layer "F.Cu") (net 4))
 (segment (start 142.24 115.96) (end 142.24 119.13635) (width 1) (layer "B.Cu") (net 4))
 (segment (start 142.24 88.65635) (end 135.5271 95.36925) (width 1) (layer "B.Cu") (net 4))
 (segment (start 142.24 84.65) (end 142.24 88.65635) (width 1) (layer "B.Cu") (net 4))
 (segment (start 129.834264 101.062086) (end 135.5271 95.36925) (width 4.5) (layer "B.Cu") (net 4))
 (segment (start 129.54 124.46) (end 129.834264 124.165736) (width 4.5) (layer "B.Cu") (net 4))
 (segment (start 134.62 125.84925) (end 130.92925 125.84925) (width 4.5) (layer "B.Cu") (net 4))
 (segment (start 142.24 119.13635) (end 135.5271 125.84925) (width 1) (layer "B.Cu") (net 4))
 (segment (start 129.834264 118.188665) (end 129.834264 101.062086) (width 4.5) (layer "B.Cu") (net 4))
 (segment (start 130.92925 125.84925) (end 129.54 124.46) (width 4.5) (layer "B.Cu") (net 4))
 (segment (start 129.834264 124.165736) (end 129.834264 118.188665) (width 4.5) (layer "B.Cu") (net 4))
 (segment (start 123.87 100.035) (end 134.3271 110.4921) (width 0.25) (layer "F.Cu") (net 6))
 (segment (start 134.3271 110.4921) (end 134.3271 116.24925) (width 0.25) (layer "F.Cu") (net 6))
 (segment (start 135.5271 121.64925) (end 135.5271 117.44925) (width 0.25) (layer "F.Cu") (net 6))
 (segment (start 134.3271 116.24925) (end 135.5271 117.44925) (width 0.25) (layer "F.Cu") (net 6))
 (segment (start 124.747133 128.778) (end 124.747133 131.792867) (width 0.25) (layer "F.Cu") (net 9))
 (segment (start 114.359928 109.22) (end 117.055101 106.524827) (width 0.25) (layer "F.Cu") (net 9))
 (segment (start 124.46 134.62) (end 125.51 135.67) (width 0.25) (layer "F.Cu") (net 9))
 (segment (start 124.46 134.62) (end 124.46 132.08) (width 0.25) (layer "F.Cu") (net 9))
 (segment (start 124.91 119.770072) (end 114.359928 109.22) (width 0.25) (layer "F.Cu") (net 9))
 (segment (start 125.51 135.67) (end 125.51 138.54) (width 0.25) (layer "F.Cu") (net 9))
 (segment (start 123.005229 104.847528) (end 123.005229 105.439598) (width 0.25) (layer "F.Cu") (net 9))
 (segment (start 125.51 139.39) (end 125.51 138.54) (width 0.25) (layer "F.Cu") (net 9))
 (segment (start 117.065804 99.385) (end 116.522195 99.928609) (width 0.25) (layer "F.Cu") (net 9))
 (segment (start 125.51 138.14) (end 125.38 138.01) (width 0.25) (layer "F.Cu") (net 9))
 (segment (start 124.747133 131.792867) (end 124.46 132.08) (width 0.25) (layer "F.Cu") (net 9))
 (segment (start 116.522195 99.928609) (end 116.522195 103.822195) (width 0.25) (layer "F.Cu") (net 9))
 (segment (start 124.91 128.615133) (end 124.91 119.770072) (width 0.25) (layer "F.Cu") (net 9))
 (segment (start 129.7 139.7) (end 125.82 139.7) (width 0.25) (layer "F.Cu") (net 9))
 (segment (start 125.428025 138.321975) (end 125.21 138.54) (width 0.25) (layer "F.Cu") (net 9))
 (segment (start 130.01 139.39) (end 129.7 139.7) (width 0.25) (layer "F.Cu") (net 9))
 (segment (start 117.055101 106.524827) (end 121.92 106.524827) (width 0.25) (layer "F.Cu") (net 9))
 (segment (start 125.82 139.7) (end 125.51 139.39) (width 0.25) (layer "F.Cu") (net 9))
 (segment (start 125.51 138.54) (end 125.51 138.14) (width 0.25) (layer "F.Cu") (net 9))
 (segment (start 123.005229 105.439598) (end 121.92 106.524827) (width 0.25) (layer "F.Cu") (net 9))
 (segment (start 124.747133 128.778) (end 124.91 128.615133) (width 0.25) (layer "F.Cu") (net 9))
 (segment (start 116.522195 103.822195) (end 117.547528 104.847528) (width 0.25) (layer "F.Cu") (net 9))
 (segment (start 130.01 138.54) (end 130.01 139.39) (width 0.25) (layer "F.Cu") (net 9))
 (segment (start 117.547528 104.847528) (end 123.005229 104.847528) (width 0.25) (layer "F.Cu") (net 9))
 (segment (start 121.92 106.524827) (end 123.005229 106.524827) (width 0.25) (layer "F.Cu") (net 9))
 (segment (start 119.97 99.385) (end 117.065804 99.385) (width 0.25) (layer "F.Cu") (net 9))
 (segment (start 123.247133 130.230865) (end 121.92 131.557998) (width 0.25) (layer "F.Cu") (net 1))
 (segment (start 116.544287 98.679132) (end 119.914132 98.679132) (width 0.25) (layer "F.Cu") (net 1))
 (segment (start 116.544287 98.119132) (end 116.544287 98.679132) (width 0.25) (layer "F.Cu") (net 1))
 (segment (start 112.04 77.47) (end 112.04 78.74) (width 0.25) (layer "F.Cu") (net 1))
 (segment (start 119.914132 98.679132) (end 119.97 98.735) (width 0.25) (layer "F.Cu") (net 1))
 (segment (start 111.929144 77.359144) (end 112.04 77.47) (width 0.25) (layer "F.Cu") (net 1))
 (segment (start 112.04 77.47) (end 108.74755 77.47) (width 0.25) (layer "F.Cu") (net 1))
 (segment (start 121.147133 129.753) (end 119.38 127.985867) (width 0.25) (layer "F.Cu") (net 1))
 (segment (start 108.671161 80.731161) (end 105.955 83.447322) (width 0.25) (layer "F.Cu") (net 1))
 (segment (start 123.247133 128.69) (end 123.247133 130.230865) (width 0.25) (layer "F.Cu") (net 1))
 (segment (start 123.247133 128.69) (end 122.184133 129.753) (width 0.25) (layer "F.Cu") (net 1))
 (segment (start 105.955 83.447322) (end 105.955 94.280305) (width 0.25) (layer "F.Cu") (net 1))
 (segment (start 108.74755 77.47) (end 108.636694 77.359144) (width 0.25) (layer "F.Cu") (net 1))
 (segment (start 119.38 127.985867) (end 119.38 124.46) (width 0.25) (layer "F.Cu") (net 1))
 (segment (start 123.87 98.735) (end 126.108182 98.735) (width 0.25) (layer "F.Cu") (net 1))
 (segment (start 108.671161 80.009503) (end 108.671161 80.731161) (width 0.25) (layer "F.Cu") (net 1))
 (segment (start 116.469287 98.044132) (end 116.544287 98.119132) (width 0.25) (layer "F.Cu") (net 1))
 (segment (start 123.210786 128.726347) (end 123.247133 128.69) (width 0.25) (layer "F.Cu") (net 1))
 (segment (start 126.108182 98.735) (end 126.135267 98.762085) (width 0.25) (layer "F.Cu") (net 1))
 (segment (start 108.636694 77.359144) (end 108.636694 79.975036) (width 0.25) (layer "F.Cu") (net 1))
 (segment (start 122.184133 129.753) (end 121.147133 129.753) (width 0.25) (layer "F.Cu") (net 1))
 (segment (start 113.383428 99.659991) (end 114.141709 98.901709) (width 0.25) (layer "F.Cu") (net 1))
 (segment (start 119.38 124.46) (end 113.383428 118.463428) (width 0.25) (layer "F.Cu") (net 1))
 (segment (start 114.141709 98.901709) (end 114.999287 98.044132) (width 0.25) (layer "F.Cu") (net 1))
 (segment (start 108.636694 79.975036) (end 108.671161 80.009503) (width 0.25) (layer "F.Cu") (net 1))
 (segment (start 105.955 94.280305) (end 110.576404 98.901709) (width 0.25) (layer "F.Cu") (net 1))
 (segment (start 108.732386 78.74) (end 108.691528 78.699142) (width 0.25) (layer "F.Cu") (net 1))
 (segment (start 113.383428 118.463428) (end 113.383428 99.659991) (width 0.25) (layer "F.Cu") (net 1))
 (segment (start 119.97 98.735) (end 123.87 98.735) (width 0.25) (layer "F.Cu") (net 1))
 (segment (start 110.576404 98.901709) (end 114.141709 98.901709) (width 0.25) (layer "F.Cu") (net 1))
 (segment (start 114.999287 98.044132) (end 116.469287 98.044132) (width 0.25) (layer "F.Cu") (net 1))
 (segment (start 128.01 135.206119) (end 128.385405 134.830714) (width 0.2) (layer "F.Cu") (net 17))
 (segment (start 128.385405 134.247662) (end 128.424205 134.208862) (width 0.2) (layer "F.Cu") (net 17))
 (segment (start 128.01 138.54) (end 128.01 135.206119) (width 0.2) (layer "F.Cu") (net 17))
 (segment (start 127.01 138.54) (end 127.01 134.63) (width 0.2) (layer "F.Cu") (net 17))
 (segment (start 128.385405 134.830714) (end 128.385405 134.247662) (width 0.2) (layer "F.Cu") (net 17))
 (segment (start 128.428817 134.208862) (end 128.428817 134.20425) (width 0.2) (layer "F.Cu") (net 17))
 (segment (start 128.424205 134.208862) (end 128.428817 134.208862) (width 0.2) (layer "F.Cu") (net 17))
 (segment (start 128.428817 134.20425) (end 128.39189 134.241177) (width 0.2) (layer "F.Cu") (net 17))
 (segment (start 112.04 91.44) (end 106.68 91.44) (width 0.2) (layer "F.Cu") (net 17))
 (via (at 106.68 91.44) (size 0.8) (drill 0.4) (layers "F.Cu" "B.Cu") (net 17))
 (via (at 128.428817 134.208862) (size 0.8) (drill 0.4) (layers "F.Cu" "B.Cu") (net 17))
 (via (at 127 134.62) (size 0.8) (drill 0.4) (layers "F.Cu" "B.Cu") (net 17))
 (segment (start 107.38 93.69005) (end 106.96995 93.28) (width 0.2) (layer "B.Cu") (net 17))
 (segment (start 107.38 94.26995) (end 107.38 93.69005) (width 0.2) (layer "B.Cu") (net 17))
 (segment (start 107.08 94.56995) (end 107.38 94.26995) (width 0.2) (layer "B.Cu") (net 17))
 (segment (start 127 134.62) (end 124.46 132.08) (width 0.2) (layer "B.Cu") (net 17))
 (segment (start 125.101491 132.721491) (end 124.46 132.08) (width 0.2) (layer "B.Cu") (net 17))
 (segment (start 106.68 93.28) (end 106.68 91.44) (width 0.2) (layer "B.Cu") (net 17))
 (segment (start 127.411138 134.208862) (end 127 134.62) (width 0.2) (layer "B.Cu") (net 17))
 (segment (start 124.46 132.08) (end 107.08 114.7) (width 0.2) (layer "B.Cu") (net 17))
 (segment (start 107.08 114.7) (end 107.08 94.56995) (width 0.2) (layer "B.Cu") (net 17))
 (segment (start 106.96995 93.28) (end 106.68 93.28) (width 0.2) (layer "B.Cu") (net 17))
 (segment (start 128.428817 134.208862) (end 127.411138 134.208862) (width 0.2) (layer "B.Cu") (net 17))
 (segment (start 128.7095 135.596011) (end 128.718767 135.586744) (width 0.2) (layer "F.Cu") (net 18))
 (segment (start 128.718767 135.586744) (end 128.718767 135.063038) (width 0.2) (layer "F.Cu") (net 18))
 (segment (start 107.95 92.71) (end 106.68 93.98) (width 0.2) (layer "F.Cu") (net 18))
 (segment (start 127.700498 134.949936) (end 127.700498 134.234491) (width 0.2) (layer "F.Cu") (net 18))
 (segment (start 128.718767 135.063038) (end 129.128817 134.652988) (width 0.2) (layer "F.Cu") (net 18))
 (segment (start 129.128817 134.652988) (end 129.128817 133.918912) (width 0.2) (layer "F.Cu") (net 18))
 (segment (start 129.136169 133.926264) (end 129.136169 134.734999) (width 0.2) (layer "F.Cu") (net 18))
 (segment (start 129.136169 134.734999) (end 128.477604 135.393564) (width 0.2) (layer "F.Cu") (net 18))
 (segment (start 127.700498 133.947231) (end 128.138867 133.508862) (width 0.2) (layer "F.Cu") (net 18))
 (segment (start 128.718767 133.508862) (end 129.136169 133.926264) (width 0.2) (layer "F.Cu") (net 18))
 (segment (start 127.51 138.54) (end 127.51 135.140434) (width 0.2) (layer "F.Cu") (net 18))
 (segment (start 128.51 135.42596) (end 128.51 138.54) (width 0.2) (layer "F.Cu") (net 18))
 (segment (start 129.128817 133.918912) (end 128.718767 133.508862) (width 0.2) (layer "F.Cu") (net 18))
 (segment (start 128.477604 135.393564) (end 128.51 135.42596) (width 0.2) (layer "F.Cu") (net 18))
 (segment (start 127.51 135.140434) (end 127.700498 134.949936) (width 0.2) (layer "F.Cu") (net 18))
 (segment (start 128.138867 133.508862) (end 128.718767 133.508862) (width 0.2) (layer "F.Cu") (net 18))
 (segment (start 127.700498 134.234491) (end 127.706549 134.22844) (width 0.2) (layer "F.Cu") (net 18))
 (segment (start 112.04 92.71) (end 107.95 92.71) (width 0.2) (layer "F.Cu") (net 18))
 (segment (start 127.700498 134.234491) (end 127.700498 133.947231) (width 0.2) (layer "F.Cu") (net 18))
 (via (at 128.7095 135.596011) (size 0.8) (drill 0.4) (layers "F.Cu" "B.Cu") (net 18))
 (via (at 106.68 93.98) (size 0.8) (drill 0.4) (layers "F.Cu" "B.Cu") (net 18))
 (segment (start 106.68 115.28995) (end 106.68 93.98) (width 0.2) (layer "B.Cu") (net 18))
 (segment (start 128.7095 135.596011) (end 128.58364 135.596011) (width 0.2) (layer "B.Cu") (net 18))
 (segment (start 128.307629 135.32) (end 126.71005 135.32) (width 0.2) (layer "B.Cu") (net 18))
 (segment (start 128.58364 135.596011) (end 128.307629 135.32) (width 0.2) (layer "B.Cu") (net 18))
 (segment (start 126.71005 135.32) (end 106.68 115.28995) (width 0.2) (layer "B.Cu") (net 18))
 (segment (start 129.54 97.288182) (end 129.481169 97.347013) (width 0.25) (layer "F.Cu") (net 5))
 (segment (start 129.54 92.73) (end 129.54 97.288182) (width 0.25) (layer "F.Cu") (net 5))
 (segment (start 110.424 131.39) (end 111.07 131.39) (width 0.25) (layer "F.Cu") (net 51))
 (segment (start 107.334264 128.300264) (end 107.334264 118.188665) (width 4.5) (layer "F.Cu") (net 51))
 (segment (start 110.424 131.39) (end 107.334264 128.300264) (width 4.5) (layer "F.Cu") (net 51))
 (segment (start 111.07 131.39) (end 111.76 132.08) (width 0.25) (layer "F.Cu") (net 51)))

